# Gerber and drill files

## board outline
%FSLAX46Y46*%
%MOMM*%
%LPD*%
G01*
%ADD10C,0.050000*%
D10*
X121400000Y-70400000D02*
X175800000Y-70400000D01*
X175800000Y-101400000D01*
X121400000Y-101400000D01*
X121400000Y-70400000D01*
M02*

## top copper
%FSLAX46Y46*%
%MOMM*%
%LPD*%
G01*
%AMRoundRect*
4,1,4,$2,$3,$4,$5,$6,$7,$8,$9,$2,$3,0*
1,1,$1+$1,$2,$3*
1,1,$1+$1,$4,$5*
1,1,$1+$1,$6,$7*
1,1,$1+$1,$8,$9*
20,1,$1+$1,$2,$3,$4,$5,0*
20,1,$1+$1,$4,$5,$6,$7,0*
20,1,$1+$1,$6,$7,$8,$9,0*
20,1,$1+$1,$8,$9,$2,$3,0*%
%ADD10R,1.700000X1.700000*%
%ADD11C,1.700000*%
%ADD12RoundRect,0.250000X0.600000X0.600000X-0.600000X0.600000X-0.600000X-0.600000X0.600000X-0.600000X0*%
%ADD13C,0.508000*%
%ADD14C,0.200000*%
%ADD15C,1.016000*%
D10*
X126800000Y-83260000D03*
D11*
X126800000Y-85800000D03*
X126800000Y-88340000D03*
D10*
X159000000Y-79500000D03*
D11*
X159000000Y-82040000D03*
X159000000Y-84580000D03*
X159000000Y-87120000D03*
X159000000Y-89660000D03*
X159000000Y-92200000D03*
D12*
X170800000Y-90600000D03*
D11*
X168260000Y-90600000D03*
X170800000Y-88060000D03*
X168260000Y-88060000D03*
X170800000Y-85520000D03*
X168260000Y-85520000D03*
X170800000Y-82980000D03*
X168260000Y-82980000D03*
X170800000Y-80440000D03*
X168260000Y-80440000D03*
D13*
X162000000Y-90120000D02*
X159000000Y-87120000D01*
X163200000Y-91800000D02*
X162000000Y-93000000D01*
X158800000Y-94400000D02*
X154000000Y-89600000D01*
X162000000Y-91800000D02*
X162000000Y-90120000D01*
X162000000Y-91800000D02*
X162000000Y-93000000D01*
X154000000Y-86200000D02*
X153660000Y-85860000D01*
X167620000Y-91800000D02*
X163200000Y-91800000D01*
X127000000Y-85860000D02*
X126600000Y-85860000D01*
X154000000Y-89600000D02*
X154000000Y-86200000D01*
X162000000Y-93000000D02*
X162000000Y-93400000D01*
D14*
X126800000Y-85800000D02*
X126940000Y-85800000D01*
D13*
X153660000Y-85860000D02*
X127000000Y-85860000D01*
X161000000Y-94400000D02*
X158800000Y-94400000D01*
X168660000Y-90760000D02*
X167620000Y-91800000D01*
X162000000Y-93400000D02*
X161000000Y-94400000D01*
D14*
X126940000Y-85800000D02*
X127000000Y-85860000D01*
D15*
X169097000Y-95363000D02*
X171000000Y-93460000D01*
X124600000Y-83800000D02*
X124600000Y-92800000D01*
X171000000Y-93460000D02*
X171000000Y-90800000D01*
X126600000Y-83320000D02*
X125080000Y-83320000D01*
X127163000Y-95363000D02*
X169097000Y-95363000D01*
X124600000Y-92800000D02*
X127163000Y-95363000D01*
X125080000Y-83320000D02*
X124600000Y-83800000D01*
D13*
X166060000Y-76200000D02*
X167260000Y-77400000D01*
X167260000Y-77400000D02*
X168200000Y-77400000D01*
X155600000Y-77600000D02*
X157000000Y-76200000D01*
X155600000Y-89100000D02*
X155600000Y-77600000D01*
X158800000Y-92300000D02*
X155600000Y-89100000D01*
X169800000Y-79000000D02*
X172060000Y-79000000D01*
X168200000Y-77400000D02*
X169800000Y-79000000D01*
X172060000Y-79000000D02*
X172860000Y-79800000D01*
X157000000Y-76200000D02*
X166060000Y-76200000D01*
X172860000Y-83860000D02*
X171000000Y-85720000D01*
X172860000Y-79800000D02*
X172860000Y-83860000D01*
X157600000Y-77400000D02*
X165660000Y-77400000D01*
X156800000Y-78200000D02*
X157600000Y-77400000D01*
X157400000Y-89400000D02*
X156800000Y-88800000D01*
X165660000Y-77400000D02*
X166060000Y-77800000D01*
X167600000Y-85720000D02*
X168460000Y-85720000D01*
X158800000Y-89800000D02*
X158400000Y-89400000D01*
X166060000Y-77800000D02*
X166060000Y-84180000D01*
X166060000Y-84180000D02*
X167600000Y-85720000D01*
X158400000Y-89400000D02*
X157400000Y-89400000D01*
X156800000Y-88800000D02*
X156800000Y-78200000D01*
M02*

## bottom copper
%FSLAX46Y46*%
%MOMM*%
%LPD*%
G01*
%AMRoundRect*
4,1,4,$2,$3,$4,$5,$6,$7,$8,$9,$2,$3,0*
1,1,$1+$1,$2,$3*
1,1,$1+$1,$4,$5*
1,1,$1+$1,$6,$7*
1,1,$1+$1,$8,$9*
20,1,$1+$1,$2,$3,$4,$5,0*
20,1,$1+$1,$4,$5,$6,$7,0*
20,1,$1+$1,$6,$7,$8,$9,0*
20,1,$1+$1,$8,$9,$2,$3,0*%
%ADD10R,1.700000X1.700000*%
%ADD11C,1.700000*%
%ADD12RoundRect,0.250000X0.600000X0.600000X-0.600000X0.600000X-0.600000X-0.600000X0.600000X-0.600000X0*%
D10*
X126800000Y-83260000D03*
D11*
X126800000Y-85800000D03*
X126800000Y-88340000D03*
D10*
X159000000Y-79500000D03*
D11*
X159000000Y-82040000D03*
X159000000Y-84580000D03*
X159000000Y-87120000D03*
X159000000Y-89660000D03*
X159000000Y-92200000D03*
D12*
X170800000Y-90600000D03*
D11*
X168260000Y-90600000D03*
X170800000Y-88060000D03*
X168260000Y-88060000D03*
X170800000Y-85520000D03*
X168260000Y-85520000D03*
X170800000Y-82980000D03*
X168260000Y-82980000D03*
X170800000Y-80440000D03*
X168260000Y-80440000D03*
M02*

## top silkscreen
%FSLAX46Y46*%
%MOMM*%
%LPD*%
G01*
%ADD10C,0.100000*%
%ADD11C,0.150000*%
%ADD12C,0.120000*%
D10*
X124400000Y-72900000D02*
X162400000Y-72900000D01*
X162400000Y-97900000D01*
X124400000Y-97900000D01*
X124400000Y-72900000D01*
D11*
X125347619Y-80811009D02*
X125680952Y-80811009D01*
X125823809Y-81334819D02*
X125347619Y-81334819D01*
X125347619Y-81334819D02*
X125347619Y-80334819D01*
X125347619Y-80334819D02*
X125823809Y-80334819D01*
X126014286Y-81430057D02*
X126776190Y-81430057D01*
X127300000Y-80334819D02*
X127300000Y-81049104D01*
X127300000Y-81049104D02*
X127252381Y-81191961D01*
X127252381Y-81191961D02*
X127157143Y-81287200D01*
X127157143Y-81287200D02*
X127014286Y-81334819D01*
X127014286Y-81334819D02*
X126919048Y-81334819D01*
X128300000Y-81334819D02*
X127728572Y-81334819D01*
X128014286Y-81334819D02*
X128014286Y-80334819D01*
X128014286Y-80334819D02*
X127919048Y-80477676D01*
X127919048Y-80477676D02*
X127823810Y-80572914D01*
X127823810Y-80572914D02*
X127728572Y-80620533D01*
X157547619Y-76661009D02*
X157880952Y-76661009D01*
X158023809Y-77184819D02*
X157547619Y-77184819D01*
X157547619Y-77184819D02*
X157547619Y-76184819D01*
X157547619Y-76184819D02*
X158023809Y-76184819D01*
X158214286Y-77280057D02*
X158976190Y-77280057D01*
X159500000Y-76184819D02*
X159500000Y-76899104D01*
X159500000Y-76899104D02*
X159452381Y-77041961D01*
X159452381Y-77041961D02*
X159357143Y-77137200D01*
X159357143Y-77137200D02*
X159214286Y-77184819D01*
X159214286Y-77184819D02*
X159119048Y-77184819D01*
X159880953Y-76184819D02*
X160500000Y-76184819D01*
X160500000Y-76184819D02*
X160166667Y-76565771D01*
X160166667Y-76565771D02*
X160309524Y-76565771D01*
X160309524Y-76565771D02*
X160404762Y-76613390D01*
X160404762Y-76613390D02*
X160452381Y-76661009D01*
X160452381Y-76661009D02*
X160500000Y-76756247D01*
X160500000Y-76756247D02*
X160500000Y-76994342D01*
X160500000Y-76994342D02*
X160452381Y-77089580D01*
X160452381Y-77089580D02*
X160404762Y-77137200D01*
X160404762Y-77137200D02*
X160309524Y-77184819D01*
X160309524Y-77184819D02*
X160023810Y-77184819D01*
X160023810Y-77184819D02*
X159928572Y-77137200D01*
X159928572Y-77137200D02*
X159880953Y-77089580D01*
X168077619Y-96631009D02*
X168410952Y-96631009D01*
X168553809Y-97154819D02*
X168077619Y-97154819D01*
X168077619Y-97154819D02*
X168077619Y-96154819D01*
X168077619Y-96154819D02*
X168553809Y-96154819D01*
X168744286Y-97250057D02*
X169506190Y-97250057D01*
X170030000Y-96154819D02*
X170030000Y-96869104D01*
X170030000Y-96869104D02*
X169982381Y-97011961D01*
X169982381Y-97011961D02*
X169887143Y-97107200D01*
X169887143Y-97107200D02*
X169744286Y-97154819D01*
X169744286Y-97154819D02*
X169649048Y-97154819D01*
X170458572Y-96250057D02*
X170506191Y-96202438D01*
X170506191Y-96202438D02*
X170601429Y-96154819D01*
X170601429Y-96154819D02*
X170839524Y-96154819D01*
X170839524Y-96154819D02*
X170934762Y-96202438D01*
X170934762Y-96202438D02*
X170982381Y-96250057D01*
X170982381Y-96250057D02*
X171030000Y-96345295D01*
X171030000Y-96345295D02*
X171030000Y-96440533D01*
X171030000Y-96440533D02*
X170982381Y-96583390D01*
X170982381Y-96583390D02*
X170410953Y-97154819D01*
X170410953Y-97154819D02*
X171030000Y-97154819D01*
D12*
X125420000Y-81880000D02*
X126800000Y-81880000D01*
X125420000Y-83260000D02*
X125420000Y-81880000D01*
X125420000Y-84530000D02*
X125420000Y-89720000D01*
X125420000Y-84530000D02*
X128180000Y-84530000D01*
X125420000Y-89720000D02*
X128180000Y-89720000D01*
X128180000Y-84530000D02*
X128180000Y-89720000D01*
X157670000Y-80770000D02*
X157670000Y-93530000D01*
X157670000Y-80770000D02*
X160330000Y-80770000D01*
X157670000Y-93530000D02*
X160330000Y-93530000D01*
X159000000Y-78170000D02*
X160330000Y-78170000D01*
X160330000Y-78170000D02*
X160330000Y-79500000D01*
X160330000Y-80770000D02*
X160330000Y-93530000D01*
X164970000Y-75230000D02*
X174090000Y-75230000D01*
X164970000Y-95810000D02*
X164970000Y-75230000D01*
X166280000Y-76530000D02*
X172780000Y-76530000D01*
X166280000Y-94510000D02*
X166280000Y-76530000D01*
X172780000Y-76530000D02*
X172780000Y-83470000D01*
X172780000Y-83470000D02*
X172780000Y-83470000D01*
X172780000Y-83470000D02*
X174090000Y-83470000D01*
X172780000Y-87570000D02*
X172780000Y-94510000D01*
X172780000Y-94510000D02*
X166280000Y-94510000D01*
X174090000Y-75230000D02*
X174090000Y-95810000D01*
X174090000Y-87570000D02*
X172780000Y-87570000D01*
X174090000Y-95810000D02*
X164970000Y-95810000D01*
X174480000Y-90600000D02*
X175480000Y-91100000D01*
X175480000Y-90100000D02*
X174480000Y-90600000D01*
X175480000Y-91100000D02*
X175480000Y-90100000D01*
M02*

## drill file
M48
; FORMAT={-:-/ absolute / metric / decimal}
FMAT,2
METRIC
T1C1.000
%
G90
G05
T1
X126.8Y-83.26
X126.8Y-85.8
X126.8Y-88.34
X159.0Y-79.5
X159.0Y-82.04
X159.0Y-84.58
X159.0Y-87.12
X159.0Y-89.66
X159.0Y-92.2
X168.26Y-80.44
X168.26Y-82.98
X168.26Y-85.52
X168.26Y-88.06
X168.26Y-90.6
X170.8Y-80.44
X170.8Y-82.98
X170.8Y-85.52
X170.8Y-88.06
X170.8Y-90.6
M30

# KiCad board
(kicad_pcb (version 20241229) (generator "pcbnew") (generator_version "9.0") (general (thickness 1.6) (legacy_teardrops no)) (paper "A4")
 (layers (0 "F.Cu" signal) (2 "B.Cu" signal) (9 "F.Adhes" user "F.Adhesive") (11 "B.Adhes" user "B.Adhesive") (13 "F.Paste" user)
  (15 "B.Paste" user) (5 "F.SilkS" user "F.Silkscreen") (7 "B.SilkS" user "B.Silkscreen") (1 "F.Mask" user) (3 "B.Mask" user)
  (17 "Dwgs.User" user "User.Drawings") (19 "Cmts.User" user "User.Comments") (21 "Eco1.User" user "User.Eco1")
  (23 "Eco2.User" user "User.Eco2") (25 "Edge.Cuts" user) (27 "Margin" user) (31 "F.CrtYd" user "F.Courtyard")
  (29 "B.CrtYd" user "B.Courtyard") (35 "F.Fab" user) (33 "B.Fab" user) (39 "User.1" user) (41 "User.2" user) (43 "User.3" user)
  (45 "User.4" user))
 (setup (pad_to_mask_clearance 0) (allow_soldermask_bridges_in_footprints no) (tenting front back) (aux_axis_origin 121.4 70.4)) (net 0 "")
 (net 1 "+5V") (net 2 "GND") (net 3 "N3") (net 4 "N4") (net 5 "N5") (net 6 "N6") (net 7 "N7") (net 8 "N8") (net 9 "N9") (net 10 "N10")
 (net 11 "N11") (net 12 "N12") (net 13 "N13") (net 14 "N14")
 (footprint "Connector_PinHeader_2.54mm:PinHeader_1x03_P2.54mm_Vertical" (layer "F.Cu") (at 126.8 83.26)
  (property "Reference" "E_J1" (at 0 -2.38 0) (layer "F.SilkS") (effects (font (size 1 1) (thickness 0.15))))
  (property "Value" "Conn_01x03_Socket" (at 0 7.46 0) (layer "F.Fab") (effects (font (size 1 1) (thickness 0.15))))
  (fp_line (start -1.38 -1.38) (end 0 -1.38) (stroke (width 0.12) (type solid)) (layer "F.SilkS"))
  (fp_line (start -1.38 0) (end -1.38 -1.38) (stroke (width 0.12) (type solid)) (layer "F.SilkS"))
  (fp_line (start -1.38 1.27) (end -1.38 6.46) (stroke (width 0.12) (type solid)) (layer "F.SilkS"))
  (fp_line (start -1.38 1.27) (end 1.38 1.27) (stroke (width 0.12) (type solid)) (layer "F.SilkS"))
  (fp_line (start -1.38 6.46) (end 1.38 6.46) (stroke (width 0.12) (type solid)) (layer "F.SilkS"))
  (fp_line (start 1.38 1.27) (end 1.38 6.46) (stroke (width 0.12) (type solid)) (layer "F.SilkS"))
  (pad "1" thru_hole rect (at 0 0) (size 1.7 1.7) (drill 1) (layers "*.Cu" "*.Mask") (remove_unused_layers no) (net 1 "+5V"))
  (pad "2" thru_hole circle (at 0 2.54) (size 1.7 1.7) (drill 1) (layers "*.Cu" "*.Mask") (remove_unused_layers no) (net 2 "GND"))
  (pad "3" thru_hole circle (at 0 5.08) (size 1.7 1.7) (drill 1) (layers "*.Cu" "*.Mask") (remove_unused_layers no) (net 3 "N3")))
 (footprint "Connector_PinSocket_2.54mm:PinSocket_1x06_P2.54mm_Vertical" (layer "F.Cu") (at 159 79.5)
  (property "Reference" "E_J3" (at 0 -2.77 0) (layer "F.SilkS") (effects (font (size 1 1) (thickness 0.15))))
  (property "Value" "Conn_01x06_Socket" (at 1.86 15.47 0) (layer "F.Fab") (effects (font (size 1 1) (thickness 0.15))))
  (fp_line (start -1.33 1.27) (end -1.33 14.03) (stroke (width 0.12) (type solid)) (layer "F.SilkS"))
  (fp_line (start -1.33 1.27) (end 1.33 1.27) (stroke (width 0.12) (type solid)) (layer "F.SilkS"))
  (fp_line (start -1.33 14.03) (end 1.33 14.03) (stroke (width 0.12) (type solid)) (layer "F.SilkS"))
  (fp_line (start 0 -1.33) (end 1.33 -1.33) (stroke (width 0.12) (type solid)) (layer "F.SilkS"))
  (fp_line (start 1.33 -1.33) (end 1.33 0) (stroke (width 0.12) (type solid)) (layer "F.SilkS"))
  (fp_line (start 1.33 1.27) (end 1.33 14.03) (stroke (width 0.12) (type solid)) (layer "F.SilkS"))
  (pad "1" thru_hole rect (at 0 0) (size 1.7 1.7) (drill 1) (layers "*.Cu" "*.Mask") (remove_unused_layers no) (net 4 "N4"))
  (pad "2" thru_hole circle (at 0 2.54) (size 1.7 1.7) (drill 1) (layers "*.Cu" "*.Mask") (remove_unused_layers no) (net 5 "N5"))
  (pad "3" thru_hole circle (at 0 5.08) (size 1.7 1.7) (drill 1) (layers "*.Cu" "*.Mask") (remove_unused_layers no) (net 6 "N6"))
  (pad "4" thru_hole circle (at 0 7.62) (size 1.7 1.7) (drill 1) (layers "*.Cu" "*.Mask") (remove_unused_layers no) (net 2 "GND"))
  (pad "5" thru_hole circle (at 0 10.16) (size 1.7 1.7) (drill 1) (layers "*.Cu" "*.Mask") (remove_unused_layers no) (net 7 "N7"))
  (pad "6" thru_hole circle (at 0 12.7) (size 1.7 1.7) (drill 1) (layers "*.Cu" "*.Mask") (remove_unused_layers no) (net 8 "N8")))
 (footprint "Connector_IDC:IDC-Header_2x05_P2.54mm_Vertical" (layer "F.Cu") (at 170.8 90.6 180)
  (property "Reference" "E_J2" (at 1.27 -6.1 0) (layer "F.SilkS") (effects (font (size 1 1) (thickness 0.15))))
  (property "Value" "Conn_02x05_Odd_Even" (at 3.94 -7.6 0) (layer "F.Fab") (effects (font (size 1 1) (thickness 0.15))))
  (fp_line (start 5.83 15.37) (end -3.29 15.37) (stroke (width 0.12) (type solid)) (layer "F.SilkS"))
  (fp_line (start 5.83 -5.21) (end 5.83 15.37) (stroke (width 0.12) (type solid)) (layer "F.SilkS"))
  (fp_line (start 4.52 14.07) (end -1.98 14.07) (stroke (width 0.12) (type solid)) (layer "F.SilkS"))
  (fp_line (start 4.52 -3.91) (end 4.52 14.07) (stroke (width 0.12) (type solid)) (layer "F.SilkS"))
  (fp_line (start -1.98 14.07) (end -1.98 7.13) (stroke (width 0.12) (type solid)) (layer "F.SilkS"))
  (fp_line (start -1.98 7.13) (end -1.98 7.13) (stroke (width 0.12) (type solid)) (layer "F.SilkS"))
  (fp_line (start -1.98 7.13) (end -3.29 7.13) (stroke (width 0.12) (type solid)) (layer "F.SilkS"))
  (fp_line (start -1.98 3.03) (end -1.98 -3.91) (stroke (width 0.12) (type solid)) (layer "F.SilkS"))
  (fp_line (start -1.98 -3.91) (end 4.52 -3.91) (stroke (width 0.12) (type solid)) (layer "F.SilkS"))
  (fp_line (start -3.29 15.37) (end -3.29 -5.21) (stroke (width 0.12) (type solid)) (layer "F.SilkS"))
  (fp_line (start -3.29 3.03) (end -1.98 3.03) (stroke (width 0.12) (type solid)) (layer "F.SilkS"))
  (fp_line (start -3.29 -5.21) (end 5.83 -5.21) (stroke (width 0.12) (type solid)) (layer "F.SilkS"))
  (fp_line (start -3.68 0) (end -4.68 -0.5) (stroke (width 0.12) (type solid)) (layer "F.SilkS"))
  (fp_line (start -4.68 0.5) (end -3.68 0) (stroke (width 0.12) (type solid)) (layer "F.SilkS"))
  (fp_line (start -4.68 -0.5) (end -4.68 0.5) (stroke (width 0.12) (type solid)) (layer "F.SilkS"))
  (pad "1" thru_hole roundrect (at 0 0 180) (size 1.7 1.7) (drill 1) (layers "*.Cu" "*.Mask") (remove_unused_layers no)
   (roundrect_rratio 0.147059) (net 1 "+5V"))
  (pad "2" thru_hole circle (at 2.54 0 180) (size 1.7 1.7) (drill 1) (layers "*.Cu" "*.Mask") (remove_unused_layers no) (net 2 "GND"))
  (pad "3" thru_hole circle (at 0 2.54 180) (size 1.7 1.7) (drill 1) (layers "*.Cu" "*.Mask") (remove_unused_layers no) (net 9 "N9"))
  (pad "4" thru_hole circle (at 2.54 2.54 180) (size 1.7 1.7) (drill 1) (layers "*.Cu" "*.Mask") (remove_unused_layers no) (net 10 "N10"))
  (pad "5" thru_hole circle (at 0 5.08 180) (size 1.7 1.7) (drill 1) (layers "*.Cu" "*.Mask") (remove_unused_layers no) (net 8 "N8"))
  (pad "6" thru_hole circle (at 2.54 5.08 180) (size 1.7 1.7) (drill 1) (layers "*.Cu" "*.Mask") (remove_unused_layers no) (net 7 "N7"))
  (pad "7" thru_hole circle (at 0 7.62 180) (size 1.7 1.7) (drill 1) (layers "*.Cu" "*.Mask") (remove_unused_layers no) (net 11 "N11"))
  (pad "8" thru_hole circle (at 2.54 7.62 180) (size 1.7 1.7) (drill 1) (layers "*.Cu" "*.Mask") (remove_unused_layers no) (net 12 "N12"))
  (pad "9" thru_hole circle (at 0 10.16 180) (size 1.7 1.7) (drill 1) (layers "*.Cu" "*.Mask") (remove_unused_layers no) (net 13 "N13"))
  (pad "10" thru_hole circle (at 2.54 10.16 180) (size 1.7 1.7) (drill 1) (layers "*.Cu" "*.Mask") (remove_unused_layers no) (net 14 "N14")))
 (gr_rect (start 124.4 72.9) (end 162.4 97.9) (stroke (width 0.1) (type default)) (fill no) (layer "F.SilkS"))
 (gr_rect (start 121.4 70.4) (end 175.8 101.4) (stroke (width 0.05) (type default)) (fill no) (layer "Edge.Cuts"))
 (segment (start 162 90.12) (end 159 87.12) (width 0.508) (layer "F.Cu") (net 2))
 (segment (start 163.2 91.8) (end 162 93) (width 0.508) (layer "F.Cu") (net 2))
 (segment (start 158.8 94.4) (end 154 89.6) (width 0.508) (layer "F.Cu") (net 2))
 (segment (start 162 91.8) (end 162 90.12) (width 0.508) (layer "F.Cu") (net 2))
 (segment (start 162 91.8) (end 162 93) (width 0.508) (layer "F.Cu") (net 2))
 (segment (start 154 86.2) (end 153.66 85.86) (width 0.508) (layer "F.Cu") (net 2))
 (segment (start 167.62 91.8) (end 163.2 91.8) (width 0.508) (layer "F.Cu") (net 2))
 (segment (start 127 85.86) (end 126.6 85.86) (width 0.508) (layer "F.Cu") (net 2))
 (segment (start 154 89.6) (end 154 86.2) (width 0.508) (layer "F.Cu") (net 2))
 (segment (start 162 93) (end 162 93.4) (width 0.508) (layer "F.Cu") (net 2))
 (segment (start 126.8 85.8) (end 126.94 85.8) (width 0.2) (layer "F.Cu") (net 2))
 (segment (start 153.66 85.86) (end 127 85.86) (width 0.508) (layer "F.Cu") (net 2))
 (segment (start 161 94.4) (end 158.8 94.4) (width 0.508) (layer "F.Cu") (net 2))
 (segment (start 168.66 90.76) (end 167.62 91.8) (width 0.508) (layer "F.Cu") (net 2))
 (segment (start 162 93.4) (end 161 94.4) (width 0.508) (layer "F.Cu") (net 2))
 (segment (start 126.94 85.8) (end 127 85.86) (width 0.2) (layer "F.Cu") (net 2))
 (segment (start 169.097 95.363) (end 171 93.46) (width 1.016) (layer "F.Cu") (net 1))
 (segment (start 124.6 83.8) (end 124.6 92.8) (width 1.016) (layer "F.Cu") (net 1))
 (segment (start 171 93.46) (end 171 90.8) (width 1.016) (layer "F.Cu") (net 1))
 (segment (start 126.6 83.32) (end 125.08 83.32) (width 1.016) (layer "F.Cu") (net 1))
 (segment (start 127.163 95.363) (end 169.097 95.363) (width 1.016) (layer "F.Cu") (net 1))
 (segment (start 124.6 92.8) (end 127.163 95.363) (width 1.016) (layer "F.Cu") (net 1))
 (segment (start 125.08 83.32) (end 124.6 83.8) (width 1.016) (layer "F.Cu") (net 1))
 (segment (start 166.06 76.2) (end 167.26 77.4) (width 0.508) (layer "F.Cu") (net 8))
 (segment (start 167.26 77.4) (end 168.2 77.4) (width 0.508) (layer "F.Cu") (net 8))
 (segment (start 155.6 77.6) (end 157 76.2) (width 0.508) (layer "F.Cu") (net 8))
 (segment (start 155.6 89.1) (end 155.6 77.6) (width 0.508) (layer "F.Cu") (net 8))
 (segment (start 158.8 92.3) (end 155.6 89.1) (width 0.508) (layer "F.Cu") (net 8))
 (segment (start 169.8 79) (end 172.06 79) (width 0.508) (layer "F.Cu") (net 8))
 (segment (start 168.2 77.4) (end 169.8 79) (width 0.508) (layer "F.Cu") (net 8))
 (segment (start 172.06 79) (end 172.86 79.8) (width 0.508) (layer "F.Cu") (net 8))
 (segment (start 157 76.2) (end 166.06 76.2) (width 0.508) (layer "F.Cu") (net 8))
 (segment (start 172.86 83.86) (end 171 85.72) (width 0.508) (layer "F.Cu") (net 8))
 (segment (start 172.86 79.8) (end 172.86 83.86) (width 0.508) (layer "F.Cu") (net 8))
 (segment (start 157.6 77.4) (end 165.66 77.4) (width 0.508) (layer "F.Cu") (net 7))
 (segment (start 156.8 78.2) (end 157.6 77.4) (width 0.508) (layer "F.Cu") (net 7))
 (segment (start 157.4 89.4) (end 156.8 88.8) (width 0.508) (layer "F.Cu") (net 7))
 (segment (start 165.66 77.4) (end 166.06 77.8) (width 0.508) (layer "F.Cu") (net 7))
 (segment (start 167.6 85.72) (end 168.46 85.72) (width 0.508) (layer "F.Cu") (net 7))
 (segment (start 158.8 89.8) (end 158.4 89.4) (width 0.508) (layer "F.Cu") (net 7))
 (segment (start 166.06 77.8) (end 166.06 84.18) (width 0.508) (layer "F.Cu") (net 7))
 (segment (start 166.06 84.18) (end 167.6 85.72) (width 0.508) (layer "F.Cu") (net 7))
 (segment (start 158.4 89.4) (end 157.4 89.4) (width 0.508) (layer "F.Cu") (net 7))
 (segment (start 156.8 88.8) (end 156.8 78.2) (width 0.508) (layer "F.Cu") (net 7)))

